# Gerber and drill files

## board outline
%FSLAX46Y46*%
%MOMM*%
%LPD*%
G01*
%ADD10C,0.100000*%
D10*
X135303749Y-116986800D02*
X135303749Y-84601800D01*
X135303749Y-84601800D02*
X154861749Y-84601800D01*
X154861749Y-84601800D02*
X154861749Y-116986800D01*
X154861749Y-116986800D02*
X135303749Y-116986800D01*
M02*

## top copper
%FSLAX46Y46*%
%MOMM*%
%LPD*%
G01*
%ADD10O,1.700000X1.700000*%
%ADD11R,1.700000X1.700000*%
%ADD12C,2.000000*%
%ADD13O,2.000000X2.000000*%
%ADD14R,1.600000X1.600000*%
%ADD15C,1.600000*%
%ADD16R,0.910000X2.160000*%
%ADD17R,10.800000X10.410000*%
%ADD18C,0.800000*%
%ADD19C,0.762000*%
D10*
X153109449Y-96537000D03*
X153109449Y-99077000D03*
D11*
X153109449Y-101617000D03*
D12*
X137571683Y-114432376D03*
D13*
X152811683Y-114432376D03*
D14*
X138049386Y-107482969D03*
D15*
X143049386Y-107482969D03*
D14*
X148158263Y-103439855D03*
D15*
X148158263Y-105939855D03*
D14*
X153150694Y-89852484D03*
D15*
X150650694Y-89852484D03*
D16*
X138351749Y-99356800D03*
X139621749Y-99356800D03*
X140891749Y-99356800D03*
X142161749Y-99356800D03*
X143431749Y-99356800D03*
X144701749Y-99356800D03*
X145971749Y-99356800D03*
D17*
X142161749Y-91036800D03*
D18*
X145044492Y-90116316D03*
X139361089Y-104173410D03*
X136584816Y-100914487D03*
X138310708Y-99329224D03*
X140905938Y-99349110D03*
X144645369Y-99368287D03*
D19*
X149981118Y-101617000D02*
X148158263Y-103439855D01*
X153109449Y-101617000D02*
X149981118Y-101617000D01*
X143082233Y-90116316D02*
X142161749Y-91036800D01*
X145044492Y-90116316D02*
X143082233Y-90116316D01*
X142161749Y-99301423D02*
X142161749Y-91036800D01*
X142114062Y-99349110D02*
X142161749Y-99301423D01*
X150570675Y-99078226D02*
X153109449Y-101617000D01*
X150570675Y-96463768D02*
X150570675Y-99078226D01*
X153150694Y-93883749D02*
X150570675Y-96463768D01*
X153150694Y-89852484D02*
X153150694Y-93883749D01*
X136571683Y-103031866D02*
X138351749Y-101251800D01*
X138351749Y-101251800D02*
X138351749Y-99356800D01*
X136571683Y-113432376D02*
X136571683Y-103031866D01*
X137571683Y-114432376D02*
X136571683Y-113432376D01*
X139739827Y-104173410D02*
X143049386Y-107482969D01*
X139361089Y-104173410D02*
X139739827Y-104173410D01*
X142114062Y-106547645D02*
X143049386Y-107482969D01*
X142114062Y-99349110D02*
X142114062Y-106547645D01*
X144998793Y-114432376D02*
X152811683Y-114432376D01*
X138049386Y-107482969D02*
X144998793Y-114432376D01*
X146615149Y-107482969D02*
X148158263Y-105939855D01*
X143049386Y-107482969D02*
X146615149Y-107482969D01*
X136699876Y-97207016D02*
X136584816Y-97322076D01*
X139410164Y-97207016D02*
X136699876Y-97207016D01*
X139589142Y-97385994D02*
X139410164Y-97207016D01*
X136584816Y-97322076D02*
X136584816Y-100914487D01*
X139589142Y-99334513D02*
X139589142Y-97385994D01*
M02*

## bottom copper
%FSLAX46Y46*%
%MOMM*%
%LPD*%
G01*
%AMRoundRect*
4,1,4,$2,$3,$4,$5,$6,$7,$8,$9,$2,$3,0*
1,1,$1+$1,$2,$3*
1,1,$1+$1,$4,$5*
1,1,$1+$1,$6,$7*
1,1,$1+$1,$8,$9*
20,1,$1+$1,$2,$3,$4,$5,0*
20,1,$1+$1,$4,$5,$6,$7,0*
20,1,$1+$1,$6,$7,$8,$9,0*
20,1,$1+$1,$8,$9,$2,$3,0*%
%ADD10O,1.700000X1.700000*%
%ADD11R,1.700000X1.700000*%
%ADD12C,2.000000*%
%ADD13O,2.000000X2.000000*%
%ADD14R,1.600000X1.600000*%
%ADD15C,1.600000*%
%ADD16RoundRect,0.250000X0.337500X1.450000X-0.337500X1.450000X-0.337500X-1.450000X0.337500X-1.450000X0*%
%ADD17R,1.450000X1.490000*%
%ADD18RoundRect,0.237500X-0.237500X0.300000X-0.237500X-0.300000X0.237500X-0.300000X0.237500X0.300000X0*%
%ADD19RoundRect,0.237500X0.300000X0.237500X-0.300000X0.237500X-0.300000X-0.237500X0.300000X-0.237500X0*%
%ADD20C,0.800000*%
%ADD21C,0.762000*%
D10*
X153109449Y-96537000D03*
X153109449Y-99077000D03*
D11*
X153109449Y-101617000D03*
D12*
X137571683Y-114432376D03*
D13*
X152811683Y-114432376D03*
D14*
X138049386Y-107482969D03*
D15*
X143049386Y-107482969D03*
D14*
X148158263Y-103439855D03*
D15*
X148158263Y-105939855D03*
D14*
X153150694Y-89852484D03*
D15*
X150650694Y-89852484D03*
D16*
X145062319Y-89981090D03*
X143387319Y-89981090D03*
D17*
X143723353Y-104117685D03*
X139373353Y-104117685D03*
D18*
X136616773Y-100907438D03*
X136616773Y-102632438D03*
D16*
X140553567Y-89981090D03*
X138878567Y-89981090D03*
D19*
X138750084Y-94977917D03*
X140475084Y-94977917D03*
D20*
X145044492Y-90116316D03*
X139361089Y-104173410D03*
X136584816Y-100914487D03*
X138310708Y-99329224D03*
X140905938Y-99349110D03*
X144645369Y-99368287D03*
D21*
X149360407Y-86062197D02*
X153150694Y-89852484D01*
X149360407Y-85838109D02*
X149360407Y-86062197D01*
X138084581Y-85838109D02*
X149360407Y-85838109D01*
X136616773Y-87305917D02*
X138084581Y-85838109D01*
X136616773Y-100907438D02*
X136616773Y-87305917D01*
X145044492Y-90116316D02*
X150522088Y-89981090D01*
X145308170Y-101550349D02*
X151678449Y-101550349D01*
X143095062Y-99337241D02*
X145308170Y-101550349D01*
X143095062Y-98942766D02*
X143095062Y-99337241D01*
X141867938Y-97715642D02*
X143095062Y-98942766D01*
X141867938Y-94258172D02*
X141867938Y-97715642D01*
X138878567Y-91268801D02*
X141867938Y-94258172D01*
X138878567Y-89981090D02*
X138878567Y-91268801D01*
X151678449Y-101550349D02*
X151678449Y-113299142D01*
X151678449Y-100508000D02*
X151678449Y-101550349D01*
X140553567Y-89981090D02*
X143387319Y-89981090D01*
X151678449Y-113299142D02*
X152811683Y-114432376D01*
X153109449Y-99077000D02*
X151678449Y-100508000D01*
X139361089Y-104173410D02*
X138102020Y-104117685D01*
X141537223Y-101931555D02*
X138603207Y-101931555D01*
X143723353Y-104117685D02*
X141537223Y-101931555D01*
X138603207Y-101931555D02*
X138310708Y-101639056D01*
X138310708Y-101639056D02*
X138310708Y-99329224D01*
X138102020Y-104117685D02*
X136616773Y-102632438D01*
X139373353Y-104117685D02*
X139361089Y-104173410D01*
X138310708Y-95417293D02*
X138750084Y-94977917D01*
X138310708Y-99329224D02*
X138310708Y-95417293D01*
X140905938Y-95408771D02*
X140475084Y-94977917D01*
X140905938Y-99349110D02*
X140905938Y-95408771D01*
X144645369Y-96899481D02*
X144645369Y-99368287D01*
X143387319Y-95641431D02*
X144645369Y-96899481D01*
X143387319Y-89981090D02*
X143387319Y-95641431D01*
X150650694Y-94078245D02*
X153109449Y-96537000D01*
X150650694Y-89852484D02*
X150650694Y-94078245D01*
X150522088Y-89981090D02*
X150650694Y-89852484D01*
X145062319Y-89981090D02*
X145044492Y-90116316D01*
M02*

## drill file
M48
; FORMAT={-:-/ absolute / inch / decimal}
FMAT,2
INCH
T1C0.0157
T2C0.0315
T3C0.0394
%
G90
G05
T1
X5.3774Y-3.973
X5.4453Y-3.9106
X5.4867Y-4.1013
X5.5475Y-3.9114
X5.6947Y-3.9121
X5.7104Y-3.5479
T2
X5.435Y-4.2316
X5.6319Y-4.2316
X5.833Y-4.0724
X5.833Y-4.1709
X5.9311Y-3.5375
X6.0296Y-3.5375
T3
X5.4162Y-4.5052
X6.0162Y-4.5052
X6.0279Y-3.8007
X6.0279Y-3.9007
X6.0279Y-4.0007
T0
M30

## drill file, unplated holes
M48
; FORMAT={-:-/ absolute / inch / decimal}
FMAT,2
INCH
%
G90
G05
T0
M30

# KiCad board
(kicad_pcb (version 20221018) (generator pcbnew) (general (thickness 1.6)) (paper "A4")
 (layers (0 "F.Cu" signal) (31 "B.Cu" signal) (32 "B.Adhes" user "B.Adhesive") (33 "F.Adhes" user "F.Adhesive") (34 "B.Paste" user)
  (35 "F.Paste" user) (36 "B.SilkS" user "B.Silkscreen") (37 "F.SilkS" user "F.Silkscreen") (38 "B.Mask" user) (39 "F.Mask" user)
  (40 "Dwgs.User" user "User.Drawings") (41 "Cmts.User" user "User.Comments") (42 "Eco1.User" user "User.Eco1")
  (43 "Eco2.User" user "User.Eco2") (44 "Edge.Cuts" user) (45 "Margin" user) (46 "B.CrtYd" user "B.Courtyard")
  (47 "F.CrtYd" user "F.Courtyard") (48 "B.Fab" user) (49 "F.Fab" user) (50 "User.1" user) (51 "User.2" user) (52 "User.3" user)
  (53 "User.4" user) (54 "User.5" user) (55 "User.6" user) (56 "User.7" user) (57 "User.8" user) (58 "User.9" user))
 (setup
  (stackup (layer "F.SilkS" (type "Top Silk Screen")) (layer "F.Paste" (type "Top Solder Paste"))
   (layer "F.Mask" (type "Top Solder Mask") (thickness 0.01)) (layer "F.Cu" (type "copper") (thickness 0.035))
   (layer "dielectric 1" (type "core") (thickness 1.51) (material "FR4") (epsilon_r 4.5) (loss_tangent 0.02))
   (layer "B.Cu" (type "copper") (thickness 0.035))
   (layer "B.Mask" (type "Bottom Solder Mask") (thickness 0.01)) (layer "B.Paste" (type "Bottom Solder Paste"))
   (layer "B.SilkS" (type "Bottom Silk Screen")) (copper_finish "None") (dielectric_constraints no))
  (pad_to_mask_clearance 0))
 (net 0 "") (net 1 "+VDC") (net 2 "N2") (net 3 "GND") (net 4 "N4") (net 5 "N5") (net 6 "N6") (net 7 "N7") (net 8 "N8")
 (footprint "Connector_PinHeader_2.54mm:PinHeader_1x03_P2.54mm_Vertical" (layer "F.Cu") (at 153.109449 101.617 180)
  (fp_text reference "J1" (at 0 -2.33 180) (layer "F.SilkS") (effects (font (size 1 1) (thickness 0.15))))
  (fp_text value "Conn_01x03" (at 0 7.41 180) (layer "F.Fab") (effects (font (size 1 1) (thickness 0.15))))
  (pad "1" thru_hole rect (at 0 0 180) (size 1.7 1.7) (drill 1) (layers "*.Cu" "*.Mask") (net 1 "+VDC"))
  (pad "2" thru_hole oval (at 0 2.54 180) (size 1.7 1.7) (drill 1) (layers "*.Cu" "*.Mask") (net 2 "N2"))
  (pad "3" thru_hole oval (at 0 5.08 180) (size 1.7 1.7) (drill 1) (layers "*.Cu" "*.Mask") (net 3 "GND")))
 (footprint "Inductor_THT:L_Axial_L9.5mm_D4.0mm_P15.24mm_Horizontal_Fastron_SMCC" (layer "F.Cu") (at 137.571683 114.432376)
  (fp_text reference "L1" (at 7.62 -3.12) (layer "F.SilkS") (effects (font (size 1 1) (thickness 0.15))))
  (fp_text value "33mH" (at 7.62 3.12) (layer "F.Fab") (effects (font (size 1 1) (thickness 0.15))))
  (pad "1" thru_hole circle (at 0 0) (size 2 2) (drill 1) (layers "*.Cu" "*.Mask") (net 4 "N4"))
  (pad "2" thru_hole oval (at 15.24 0) (size 2 2) (drill 1) (layers "*.Cu" "*.Mask") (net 2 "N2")))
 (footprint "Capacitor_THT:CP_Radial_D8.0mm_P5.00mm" (layer "F.Cu") (at 138.049386 107.482969)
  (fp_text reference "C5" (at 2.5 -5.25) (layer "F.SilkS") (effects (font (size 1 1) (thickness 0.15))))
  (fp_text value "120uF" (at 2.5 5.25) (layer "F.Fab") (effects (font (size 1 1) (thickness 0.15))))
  (pad "1" thru_hole rect (at 0 0) (size 1.6 1.6) (drill 0.8) (layers "*.Cu" "*.Mask") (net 2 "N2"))
  (pad "2" thru_hole circle (at 5 0) (size 1.6 1.6) (drill 0.8) (layers "*.Cu" "*.Mask") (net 3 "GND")))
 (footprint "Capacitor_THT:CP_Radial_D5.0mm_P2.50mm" (layer "F.Cu") (at 148.158263 103.439855 -90)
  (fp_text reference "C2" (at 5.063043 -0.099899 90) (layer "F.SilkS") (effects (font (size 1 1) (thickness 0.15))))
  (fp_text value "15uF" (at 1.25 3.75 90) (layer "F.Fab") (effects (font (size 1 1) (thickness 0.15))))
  (pad "1" thru_hole rect (at 0 0 270) (size 1.6 1.6) (drill 0.8) (layers "*.Cu" "*.Mask") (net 1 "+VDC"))
  (pad "2" thru_hole circle (at 2.5 0 270) (size 1.6 1.6) (drill 0.8) (layers "*.Cu" "*.Mask") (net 3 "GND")))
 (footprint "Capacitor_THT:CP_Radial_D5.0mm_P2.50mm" (layer "F.Cu") (at 153.150694 89.852484 180)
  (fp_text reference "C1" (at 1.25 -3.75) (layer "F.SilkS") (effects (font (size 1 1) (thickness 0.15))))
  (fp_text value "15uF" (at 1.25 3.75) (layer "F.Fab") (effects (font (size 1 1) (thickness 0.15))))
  (pad "1" thru_hole rect (at 0 0 180) (size 1.6 1.6) (drill 0.8) (layers "*.Cu" "*.Mask") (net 1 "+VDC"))
  (pad "2" thru_hole circle (at 2.5 0 180) (size 1.6 1.6) (drill 0.8) (layers "*.Cu" "*.Mask") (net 3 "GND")))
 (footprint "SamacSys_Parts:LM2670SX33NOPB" (layer "F.Cu") (at 142.161749 91.5868 -90)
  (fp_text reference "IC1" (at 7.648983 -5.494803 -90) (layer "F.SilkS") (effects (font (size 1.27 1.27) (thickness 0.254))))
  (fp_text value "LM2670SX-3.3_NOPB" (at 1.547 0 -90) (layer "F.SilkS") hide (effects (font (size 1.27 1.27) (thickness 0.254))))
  (pad "1" smd rect (at 7.77 3.81) (size 0.91 2.16) (layers "F.Cu" "F.Paste" "F.Mask") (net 4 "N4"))
  (pad "2" smd rect (at 7.77 2.54) (size 0.91 2.16) (layers "F.Cu" "F.Paste" "F.Mask") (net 1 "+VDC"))
  (pad "3" smd rect (at 7.77 1.27) (size 0.91 2.16) (layers "F.Cu" "F.Paste" "F.Mask") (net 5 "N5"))
  (pad "4" smd rect (at 7.77 0) (size 0.91 2.16) (layers "F.Cu" "F.Paste" "F.Mask") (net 3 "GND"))
  (pad "5" smd rect (at 7.77 -1.27) (size 0.91 2.16) (layers "F.Cu" "F.Paste" "F.Mask") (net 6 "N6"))
  (pad "6" smd rect (at 7.77 -2.54) (size 0.91 2.16) (layers "F.Cu" "F.Paste" "F.Mask") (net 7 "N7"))
  (pad "7" smd rect (at 7.77 -3.81) (size 0.91 2.16) (layers "F.Cu" "F.Paste" "F.Mask") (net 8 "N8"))
  (pad "8" smd rect (at -0.55 0 270) (size 10.41 10.8) (layers "F.Cu" "F.Paste" "F.Mask") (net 3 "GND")))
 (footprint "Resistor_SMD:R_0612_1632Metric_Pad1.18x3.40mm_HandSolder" (layer "B.Cu") (at 144.224819 89.98109 180)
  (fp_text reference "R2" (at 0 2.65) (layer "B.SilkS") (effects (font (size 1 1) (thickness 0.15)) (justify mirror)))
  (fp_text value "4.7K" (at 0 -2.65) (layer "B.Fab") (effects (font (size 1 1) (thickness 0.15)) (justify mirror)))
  (pad "1" smd roundrect (at -0.8375 0 180) (size 1.175 3.4) (layers "B.Cu" "B.Paste" "B.Mask") (roundrect_rratio 0.2127659574)
   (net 3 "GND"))
  (pad "2" smd roundrect (at 0.8375 0 180) (size 1.175 3.4) (layers "B.Cu" "B.Paste" "B.Mask") (roundrect_rratio 0.2127659574) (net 7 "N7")))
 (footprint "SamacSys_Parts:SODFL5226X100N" (layer "B.Cu") (at 141.548353 104.117685 180)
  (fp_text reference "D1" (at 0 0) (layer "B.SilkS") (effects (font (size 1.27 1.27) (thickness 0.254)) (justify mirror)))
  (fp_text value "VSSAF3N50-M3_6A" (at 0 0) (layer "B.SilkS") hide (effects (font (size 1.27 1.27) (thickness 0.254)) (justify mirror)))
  (pad "1" smd rect (at -2.175 0 180) (size 1.45 1.49) (layers "B.Cu" "B.Paste" "B.Mask") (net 4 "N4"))
  (pad "2" smd rect (at 2.175 0 180) (size 1.45 1.49) (layers "B.Cu" "B.Paste" "B.Mask") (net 3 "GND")))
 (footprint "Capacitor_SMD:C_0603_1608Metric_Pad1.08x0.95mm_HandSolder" (layer "B.Cu") (at 136.616773 101.769938 -90)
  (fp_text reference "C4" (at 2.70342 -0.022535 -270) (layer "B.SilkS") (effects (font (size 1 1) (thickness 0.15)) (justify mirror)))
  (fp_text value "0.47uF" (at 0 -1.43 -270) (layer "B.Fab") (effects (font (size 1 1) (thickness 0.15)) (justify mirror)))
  (pad "1" smd roundrect (at -0.8625 0 270) (size 1.075 0.95) (layers "B.Cu" "B.Paste" "B.Mask") (roundrect_rratio 0.25) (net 1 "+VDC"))
  (pad "2" smd roundrect (at 0.8625 0 270) (size 1.075 0.95) (layers "B.Cu" "B.Paste" "B.Mask") (roundrect_rratio 0.25) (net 3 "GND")))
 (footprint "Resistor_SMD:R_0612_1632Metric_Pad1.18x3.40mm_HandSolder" (layer "B.Cu") (at 139.716067 89.98109 180)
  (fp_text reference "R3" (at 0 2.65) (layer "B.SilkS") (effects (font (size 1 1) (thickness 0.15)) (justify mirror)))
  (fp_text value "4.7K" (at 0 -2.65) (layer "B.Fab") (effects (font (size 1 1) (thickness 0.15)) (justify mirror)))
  (pad "1" smd roundrect (at -0.8375 0 180) (size 1.175 3.4) (layers "B.Cu" "B.Paste" "B.Mask") (roundrect_rratio 0.2127659574) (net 7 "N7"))
  (pad "2" smd roundrect (at 0.8375 0 180) (size 1.175 3.4) (layers "B.Cu" "B.Paste" "B.Mask") (roundrect_rratio 0.2127659574) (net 2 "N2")))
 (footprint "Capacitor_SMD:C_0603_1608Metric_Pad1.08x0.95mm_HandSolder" (layer "B.Cu") (at 139.612584 94.977917 180)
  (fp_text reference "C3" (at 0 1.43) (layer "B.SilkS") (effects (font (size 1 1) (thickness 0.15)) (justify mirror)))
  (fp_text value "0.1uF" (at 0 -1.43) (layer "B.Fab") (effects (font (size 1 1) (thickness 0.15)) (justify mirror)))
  (pad "1" smd roundrect (at -0.8625 0 180) (size 1.075 0.95) (layers "B.Cu" "B.Paste" "B.Mask") (roundrect_rratio 0.25) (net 5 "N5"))
  (pad "2" smd roundrect (at 0.8625 0 180) (size 1.075 0.95) (layers "B.Cu" "B.Paste" "B.Mask") (roundrect_rratio 0.25) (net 4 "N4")))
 (gr_line (start 135.303749 116.9868) (end 135.303749 84.6018) (stroke (width 0.1) (type solid)) (layer "Edge.Cuts"))
 (gr_line (start 135.303749 84.6018) (end 154.861749 84.6018) (stroke (width 0.1) (type solid)) (layer "Edge.Cuts"))
 (gr_line (start 154.861749 84.6018) (end 154.861749 116.9868) (stroke (width 0.1) (type default)) (layer "Edge.Cuts"))
 (gr_line (start 154.861749 116.9868) (end 135.303749 116.9868) (stroke (width 0.1) (type default)) (layer "Edge.Cuts"))
 (segment (start 150.570675 96.463768) (end 150.570675 99.078226) (width 0.762) (layer "F.Cu") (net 1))
 (segment (start 136.584816 97.322076) (end 136.584816 100.914487) (width 0.762) (layer "F.Cu") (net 1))
 (segment (start 153.150694 89.852484) (end 153.150694 93.883749) (width 0.762) (layer "F.Cu") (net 1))
 (segment (start 139.589142 99.334513) (end 139.589142 97.385994) (width 0.762) (layer "F.Cu") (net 1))
 (segment (start 139.410164 97.207016) (end 136.699876 97.207016) (width 0.762) (layer "F.Cu") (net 1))
 (segment (start 153.109449 101.617) (end 149.981118 101.617) (width 0.762) (layer "F.Cu") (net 1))
 (segment (start 136.699876 97.207016) (end 136.584816 97.322076) (width 0.762) (layer "F.Cu") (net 1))
 (segment (start 150.570675 99.078226) (end 153.109449 101.617) (width 0.762) (layer "F.Cu") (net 1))
 (segment (start 153.150694 93.883749) (end 150.570675 96.463768) (width 0.762) (layer "F.Cu") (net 1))
 (segment (start 149.981118 101.617) (end 148.158263 103.439855) (width 0.762) (layer "F.Cu") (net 1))
 (segment (start 139.589142 97.385994) (end 139.410164 97.207016) (width 0.762) (layer "F.Cu") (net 1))
 (via (at 136.584816 100.914487) (size 0.8) (drill 0.4) (layers "F.Cu" "B.Cu") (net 1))
 (segment (start 136.616773 100.907438) (end 136.616773 87.305917) (width 0.762) (layer "B.Cu") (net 1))
 (segment (start 149.360407 85.838109) (end 149.360407 86.062197) (width 0.762) (layer "B.Cu") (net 1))
 (segment (start 136.616773 87.305917) (end 138.084581 85.838109) (width 0.762) (layer "B.Cu") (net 1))
 (segment (start 138.084581 85.838109) (end 149.360407 85.838109) (width 0.762) (layer "B.Cu") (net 1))
 (segment (start 149.360407 86.062197) (end 153.150694 89.852484) (width 0.762) (layer "B.Cu") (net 1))
 (segment (start 142.114062 99.34911) (end 142.161749 99.301423) (width 0.762) (layer "F.Cu") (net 3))
 (segment (start 143.049386 107.482969) (end 146.615149 107.482969) (width 0.762) (layer "F.Cu") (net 3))
 (segment (start 142.114062 106.547645) (end 143.049386 107.482969) (width 0.762) (layer "F.Cu") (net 3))
 (segment (start 142.161749 99.301423) (end 142.161749 91.0368) (width 0.762) (layer "F.Cu") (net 3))
 (segment (start 145.044492 90.116316) (end 143.082233 90.116316) (width 0.762) (layer "F.Cu") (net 3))
 (segment (start 142.114062 99.34911) (end 142.114062 106.547645) (width 0.762) (layer "F.Cu") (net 3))
 (segment (start 146.615149 107.482969) (end 148.158263 105.939855) (width 0.762) (layer "F.Cu") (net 3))
 (segment (start 139.361089 104.17341) (end 139.739827 104.17341) (width 0.762) (layer "F.Cu") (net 3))
 (segment (start 139.739827 104.17341) (end 143.049386 107.482969) (width 0.762) (layer "F.Cu") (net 3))
 (segment (start 143.082233 90.116316) (end 142.161749 91.0368) (width 0.762) (layer "F.Cu") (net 3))
 (via (at 145.044492 90.116316) (size 0.8) (drill 0.4) (layers "F.Cu" "B.Cu") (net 3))
 (via (at 139.361089 104.17341) (size 0.8) (drill 0.4) (layers "F.Cu" "B.Cu") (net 3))
 (segment (start 145.062319 89.98109) (end 145.044492 90.116316) (width 0.762) (layer "B.Cu") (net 3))
 (segment (start 150.650694 89.852484) (end 150.650694 94.078245) (width 0.762) (layer "B.Cu") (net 3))
 (segment (start 150.522088 89.98109) (end 150.650694 89.852484) (width 0.762) (layer "B.Cu") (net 3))
 (segment (start 150.650694 94.078245) (end 153.109449 96.537) (width 0.762) (layer "B.Cu") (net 3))
 (segment (start 138.10202 104.117685) (end 136.616773 102.632438) (width 0.762) (layer "B.Cu") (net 3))
 (segment (start 139.361089 104.17341) (end 138.10202 104.117685) (width 0.762) (layer "B.Cu") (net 3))
 (segment (start 145.044492 90.116316) (end 150.522088 89.98109) (width 0.762) (layer "B.Cu") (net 3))
 (segment (start 139.373353 104.117685) (end 139.361089 104.17341) (width 0.762) (layer "B.Cu") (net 3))
 (via (at 140.905938 99.34911) (size 0.8) (drill 0.4) (layers "F.Cu" "B.Cu") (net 5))
 (segment (start 140.905938 95.408771) (end 140.475084 94.977917) (width 0.762) (layer "B.Cu") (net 5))
 (segment (start 140.905938 99.34911) (end 140.905938 95.408771) (width 0.762) (layer "B.Cu") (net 5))
 (segment (start 136.571683 113.432376) (end 136.571683 103.031866) (width 0.762) (layer "F.Cu") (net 4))
 (segment (start 138.351749 101.2518) (end 138.351749 99.3568) (width 0.762) (layer "F.Cu") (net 4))
 (segment (start 136.571683 103.031866) (end 138.351749 101.2518) (width 0.762) (layer "F.Cu") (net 4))
 (segment (start 137.571683 114.432376) (end 136.571683 113.432376) (width 0.762) (layer "F.Cu") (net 4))
 (via (at 138.310708 99.329224) (size 0.8) (drill 0.4) (layers "F.Cu" "B.Cu") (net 4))
 (segment (start 138.310708 101.639056) (end 138.310708 99.329224) (width 0.762) (layer "B.Cu") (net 4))
 (segment (start 138.310708 95.417293) (end 138.750084 94.977917) (width 0.762) (layer "B.Cu") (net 4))
 (segment (start 143.723353 104.117685) (end 141.537223 101.931555) (width 0.762) (layer "B.Cu") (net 4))
 (segment (start 138.603207 101.931555) (end 138.310708 101.639056) (width 0.762) (layer "B.Cu") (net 4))
 (segment (start 141.537223 101.931555) (end 138.603207 101.931555) (width 0.762) (layer "B.Cu") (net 4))
 (segment (start 138.310708 99.329224) (end 138.310708 95.417293) (width 0.762) (layer "B.Cu") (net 4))
 (segment (start 144.998793 114.432376) (end 152.811683 114.432376) (width 0.762) (layer "F.Cu") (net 2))
 (segment (start 138.049386 107.482969) (end 144.998793 114.432376) (width 0.762) (layer "F.Cu") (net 2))
 (segment (start 151.678449 101.550349) (end 151.678449 113.299142) (width 0.762) (layer "B.Cu") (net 2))
 (segment (start 143.095062 98.942766) (end 143.095062 99.337241) (width 0.762) (layer "B.Cu") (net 2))
 (segment (start 141.867938 94.258172) (end 141.867938 97.715642) (width 0.762) (layer "B.Cu") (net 2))
 (segment (start 138.878567 91.268801) (end 141.867938 94.258172) (width 0.762) (layer "B.Cu") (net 2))
 (segment (start 145.30817 101.550349) (end 151.678449 101.550349) (width 0.762) (layer "B.Cu") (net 2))
 (segment (start 153.109449 99.077) (end 151.678449 100.508) (width 0.762) (layer "B.Cu") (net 2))
 (segment (start 143.095062 99.337241) (end 145.30817 101.550349) (width 0.762) (layer "B.Cu") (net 2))
 (segment (start 138.878567 89.98109) (end 138.878567 91.268801) (width 0.762) (layer "B.Cu") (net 2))
 (segment (start 151.678449 113.299142) (end 152.811683 114.432376) (width 0.762) (layer "B.Cu") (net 2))
 (segment (start 141.867938 97.715642) (end 143.095062 98.942766) (width 0.762) (layer "B.Cu") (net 2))
 (segment (start 151.678449 100.508) (end 151.678449 101.550349) (width 0.762) (layer "B.Cu") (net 2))
 (via (at 144.645369 99.368287) (size 0.8) (drill 0.4) (layers "F.Cu" "B.Cu") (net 7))
 (segment (start 144.645369 96.899481) (end 144.645369 99.368287) (width 0.762) (layer "B.Cu") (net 7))
 (segment (start 140.553567 89.98109) (end 143.387319 89.98109) (width 0.762) (layer "B.Cu") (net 7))
 (segment (start 143.387319 95.641431) (end 144.645369 96.899481) (width 0.762) (layer "B.Cu") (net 7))
 (segment (start 143.387319 89.98109) (end 143.387319 95.641431) (width 0.762) (layer "B.Cu") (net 7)))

